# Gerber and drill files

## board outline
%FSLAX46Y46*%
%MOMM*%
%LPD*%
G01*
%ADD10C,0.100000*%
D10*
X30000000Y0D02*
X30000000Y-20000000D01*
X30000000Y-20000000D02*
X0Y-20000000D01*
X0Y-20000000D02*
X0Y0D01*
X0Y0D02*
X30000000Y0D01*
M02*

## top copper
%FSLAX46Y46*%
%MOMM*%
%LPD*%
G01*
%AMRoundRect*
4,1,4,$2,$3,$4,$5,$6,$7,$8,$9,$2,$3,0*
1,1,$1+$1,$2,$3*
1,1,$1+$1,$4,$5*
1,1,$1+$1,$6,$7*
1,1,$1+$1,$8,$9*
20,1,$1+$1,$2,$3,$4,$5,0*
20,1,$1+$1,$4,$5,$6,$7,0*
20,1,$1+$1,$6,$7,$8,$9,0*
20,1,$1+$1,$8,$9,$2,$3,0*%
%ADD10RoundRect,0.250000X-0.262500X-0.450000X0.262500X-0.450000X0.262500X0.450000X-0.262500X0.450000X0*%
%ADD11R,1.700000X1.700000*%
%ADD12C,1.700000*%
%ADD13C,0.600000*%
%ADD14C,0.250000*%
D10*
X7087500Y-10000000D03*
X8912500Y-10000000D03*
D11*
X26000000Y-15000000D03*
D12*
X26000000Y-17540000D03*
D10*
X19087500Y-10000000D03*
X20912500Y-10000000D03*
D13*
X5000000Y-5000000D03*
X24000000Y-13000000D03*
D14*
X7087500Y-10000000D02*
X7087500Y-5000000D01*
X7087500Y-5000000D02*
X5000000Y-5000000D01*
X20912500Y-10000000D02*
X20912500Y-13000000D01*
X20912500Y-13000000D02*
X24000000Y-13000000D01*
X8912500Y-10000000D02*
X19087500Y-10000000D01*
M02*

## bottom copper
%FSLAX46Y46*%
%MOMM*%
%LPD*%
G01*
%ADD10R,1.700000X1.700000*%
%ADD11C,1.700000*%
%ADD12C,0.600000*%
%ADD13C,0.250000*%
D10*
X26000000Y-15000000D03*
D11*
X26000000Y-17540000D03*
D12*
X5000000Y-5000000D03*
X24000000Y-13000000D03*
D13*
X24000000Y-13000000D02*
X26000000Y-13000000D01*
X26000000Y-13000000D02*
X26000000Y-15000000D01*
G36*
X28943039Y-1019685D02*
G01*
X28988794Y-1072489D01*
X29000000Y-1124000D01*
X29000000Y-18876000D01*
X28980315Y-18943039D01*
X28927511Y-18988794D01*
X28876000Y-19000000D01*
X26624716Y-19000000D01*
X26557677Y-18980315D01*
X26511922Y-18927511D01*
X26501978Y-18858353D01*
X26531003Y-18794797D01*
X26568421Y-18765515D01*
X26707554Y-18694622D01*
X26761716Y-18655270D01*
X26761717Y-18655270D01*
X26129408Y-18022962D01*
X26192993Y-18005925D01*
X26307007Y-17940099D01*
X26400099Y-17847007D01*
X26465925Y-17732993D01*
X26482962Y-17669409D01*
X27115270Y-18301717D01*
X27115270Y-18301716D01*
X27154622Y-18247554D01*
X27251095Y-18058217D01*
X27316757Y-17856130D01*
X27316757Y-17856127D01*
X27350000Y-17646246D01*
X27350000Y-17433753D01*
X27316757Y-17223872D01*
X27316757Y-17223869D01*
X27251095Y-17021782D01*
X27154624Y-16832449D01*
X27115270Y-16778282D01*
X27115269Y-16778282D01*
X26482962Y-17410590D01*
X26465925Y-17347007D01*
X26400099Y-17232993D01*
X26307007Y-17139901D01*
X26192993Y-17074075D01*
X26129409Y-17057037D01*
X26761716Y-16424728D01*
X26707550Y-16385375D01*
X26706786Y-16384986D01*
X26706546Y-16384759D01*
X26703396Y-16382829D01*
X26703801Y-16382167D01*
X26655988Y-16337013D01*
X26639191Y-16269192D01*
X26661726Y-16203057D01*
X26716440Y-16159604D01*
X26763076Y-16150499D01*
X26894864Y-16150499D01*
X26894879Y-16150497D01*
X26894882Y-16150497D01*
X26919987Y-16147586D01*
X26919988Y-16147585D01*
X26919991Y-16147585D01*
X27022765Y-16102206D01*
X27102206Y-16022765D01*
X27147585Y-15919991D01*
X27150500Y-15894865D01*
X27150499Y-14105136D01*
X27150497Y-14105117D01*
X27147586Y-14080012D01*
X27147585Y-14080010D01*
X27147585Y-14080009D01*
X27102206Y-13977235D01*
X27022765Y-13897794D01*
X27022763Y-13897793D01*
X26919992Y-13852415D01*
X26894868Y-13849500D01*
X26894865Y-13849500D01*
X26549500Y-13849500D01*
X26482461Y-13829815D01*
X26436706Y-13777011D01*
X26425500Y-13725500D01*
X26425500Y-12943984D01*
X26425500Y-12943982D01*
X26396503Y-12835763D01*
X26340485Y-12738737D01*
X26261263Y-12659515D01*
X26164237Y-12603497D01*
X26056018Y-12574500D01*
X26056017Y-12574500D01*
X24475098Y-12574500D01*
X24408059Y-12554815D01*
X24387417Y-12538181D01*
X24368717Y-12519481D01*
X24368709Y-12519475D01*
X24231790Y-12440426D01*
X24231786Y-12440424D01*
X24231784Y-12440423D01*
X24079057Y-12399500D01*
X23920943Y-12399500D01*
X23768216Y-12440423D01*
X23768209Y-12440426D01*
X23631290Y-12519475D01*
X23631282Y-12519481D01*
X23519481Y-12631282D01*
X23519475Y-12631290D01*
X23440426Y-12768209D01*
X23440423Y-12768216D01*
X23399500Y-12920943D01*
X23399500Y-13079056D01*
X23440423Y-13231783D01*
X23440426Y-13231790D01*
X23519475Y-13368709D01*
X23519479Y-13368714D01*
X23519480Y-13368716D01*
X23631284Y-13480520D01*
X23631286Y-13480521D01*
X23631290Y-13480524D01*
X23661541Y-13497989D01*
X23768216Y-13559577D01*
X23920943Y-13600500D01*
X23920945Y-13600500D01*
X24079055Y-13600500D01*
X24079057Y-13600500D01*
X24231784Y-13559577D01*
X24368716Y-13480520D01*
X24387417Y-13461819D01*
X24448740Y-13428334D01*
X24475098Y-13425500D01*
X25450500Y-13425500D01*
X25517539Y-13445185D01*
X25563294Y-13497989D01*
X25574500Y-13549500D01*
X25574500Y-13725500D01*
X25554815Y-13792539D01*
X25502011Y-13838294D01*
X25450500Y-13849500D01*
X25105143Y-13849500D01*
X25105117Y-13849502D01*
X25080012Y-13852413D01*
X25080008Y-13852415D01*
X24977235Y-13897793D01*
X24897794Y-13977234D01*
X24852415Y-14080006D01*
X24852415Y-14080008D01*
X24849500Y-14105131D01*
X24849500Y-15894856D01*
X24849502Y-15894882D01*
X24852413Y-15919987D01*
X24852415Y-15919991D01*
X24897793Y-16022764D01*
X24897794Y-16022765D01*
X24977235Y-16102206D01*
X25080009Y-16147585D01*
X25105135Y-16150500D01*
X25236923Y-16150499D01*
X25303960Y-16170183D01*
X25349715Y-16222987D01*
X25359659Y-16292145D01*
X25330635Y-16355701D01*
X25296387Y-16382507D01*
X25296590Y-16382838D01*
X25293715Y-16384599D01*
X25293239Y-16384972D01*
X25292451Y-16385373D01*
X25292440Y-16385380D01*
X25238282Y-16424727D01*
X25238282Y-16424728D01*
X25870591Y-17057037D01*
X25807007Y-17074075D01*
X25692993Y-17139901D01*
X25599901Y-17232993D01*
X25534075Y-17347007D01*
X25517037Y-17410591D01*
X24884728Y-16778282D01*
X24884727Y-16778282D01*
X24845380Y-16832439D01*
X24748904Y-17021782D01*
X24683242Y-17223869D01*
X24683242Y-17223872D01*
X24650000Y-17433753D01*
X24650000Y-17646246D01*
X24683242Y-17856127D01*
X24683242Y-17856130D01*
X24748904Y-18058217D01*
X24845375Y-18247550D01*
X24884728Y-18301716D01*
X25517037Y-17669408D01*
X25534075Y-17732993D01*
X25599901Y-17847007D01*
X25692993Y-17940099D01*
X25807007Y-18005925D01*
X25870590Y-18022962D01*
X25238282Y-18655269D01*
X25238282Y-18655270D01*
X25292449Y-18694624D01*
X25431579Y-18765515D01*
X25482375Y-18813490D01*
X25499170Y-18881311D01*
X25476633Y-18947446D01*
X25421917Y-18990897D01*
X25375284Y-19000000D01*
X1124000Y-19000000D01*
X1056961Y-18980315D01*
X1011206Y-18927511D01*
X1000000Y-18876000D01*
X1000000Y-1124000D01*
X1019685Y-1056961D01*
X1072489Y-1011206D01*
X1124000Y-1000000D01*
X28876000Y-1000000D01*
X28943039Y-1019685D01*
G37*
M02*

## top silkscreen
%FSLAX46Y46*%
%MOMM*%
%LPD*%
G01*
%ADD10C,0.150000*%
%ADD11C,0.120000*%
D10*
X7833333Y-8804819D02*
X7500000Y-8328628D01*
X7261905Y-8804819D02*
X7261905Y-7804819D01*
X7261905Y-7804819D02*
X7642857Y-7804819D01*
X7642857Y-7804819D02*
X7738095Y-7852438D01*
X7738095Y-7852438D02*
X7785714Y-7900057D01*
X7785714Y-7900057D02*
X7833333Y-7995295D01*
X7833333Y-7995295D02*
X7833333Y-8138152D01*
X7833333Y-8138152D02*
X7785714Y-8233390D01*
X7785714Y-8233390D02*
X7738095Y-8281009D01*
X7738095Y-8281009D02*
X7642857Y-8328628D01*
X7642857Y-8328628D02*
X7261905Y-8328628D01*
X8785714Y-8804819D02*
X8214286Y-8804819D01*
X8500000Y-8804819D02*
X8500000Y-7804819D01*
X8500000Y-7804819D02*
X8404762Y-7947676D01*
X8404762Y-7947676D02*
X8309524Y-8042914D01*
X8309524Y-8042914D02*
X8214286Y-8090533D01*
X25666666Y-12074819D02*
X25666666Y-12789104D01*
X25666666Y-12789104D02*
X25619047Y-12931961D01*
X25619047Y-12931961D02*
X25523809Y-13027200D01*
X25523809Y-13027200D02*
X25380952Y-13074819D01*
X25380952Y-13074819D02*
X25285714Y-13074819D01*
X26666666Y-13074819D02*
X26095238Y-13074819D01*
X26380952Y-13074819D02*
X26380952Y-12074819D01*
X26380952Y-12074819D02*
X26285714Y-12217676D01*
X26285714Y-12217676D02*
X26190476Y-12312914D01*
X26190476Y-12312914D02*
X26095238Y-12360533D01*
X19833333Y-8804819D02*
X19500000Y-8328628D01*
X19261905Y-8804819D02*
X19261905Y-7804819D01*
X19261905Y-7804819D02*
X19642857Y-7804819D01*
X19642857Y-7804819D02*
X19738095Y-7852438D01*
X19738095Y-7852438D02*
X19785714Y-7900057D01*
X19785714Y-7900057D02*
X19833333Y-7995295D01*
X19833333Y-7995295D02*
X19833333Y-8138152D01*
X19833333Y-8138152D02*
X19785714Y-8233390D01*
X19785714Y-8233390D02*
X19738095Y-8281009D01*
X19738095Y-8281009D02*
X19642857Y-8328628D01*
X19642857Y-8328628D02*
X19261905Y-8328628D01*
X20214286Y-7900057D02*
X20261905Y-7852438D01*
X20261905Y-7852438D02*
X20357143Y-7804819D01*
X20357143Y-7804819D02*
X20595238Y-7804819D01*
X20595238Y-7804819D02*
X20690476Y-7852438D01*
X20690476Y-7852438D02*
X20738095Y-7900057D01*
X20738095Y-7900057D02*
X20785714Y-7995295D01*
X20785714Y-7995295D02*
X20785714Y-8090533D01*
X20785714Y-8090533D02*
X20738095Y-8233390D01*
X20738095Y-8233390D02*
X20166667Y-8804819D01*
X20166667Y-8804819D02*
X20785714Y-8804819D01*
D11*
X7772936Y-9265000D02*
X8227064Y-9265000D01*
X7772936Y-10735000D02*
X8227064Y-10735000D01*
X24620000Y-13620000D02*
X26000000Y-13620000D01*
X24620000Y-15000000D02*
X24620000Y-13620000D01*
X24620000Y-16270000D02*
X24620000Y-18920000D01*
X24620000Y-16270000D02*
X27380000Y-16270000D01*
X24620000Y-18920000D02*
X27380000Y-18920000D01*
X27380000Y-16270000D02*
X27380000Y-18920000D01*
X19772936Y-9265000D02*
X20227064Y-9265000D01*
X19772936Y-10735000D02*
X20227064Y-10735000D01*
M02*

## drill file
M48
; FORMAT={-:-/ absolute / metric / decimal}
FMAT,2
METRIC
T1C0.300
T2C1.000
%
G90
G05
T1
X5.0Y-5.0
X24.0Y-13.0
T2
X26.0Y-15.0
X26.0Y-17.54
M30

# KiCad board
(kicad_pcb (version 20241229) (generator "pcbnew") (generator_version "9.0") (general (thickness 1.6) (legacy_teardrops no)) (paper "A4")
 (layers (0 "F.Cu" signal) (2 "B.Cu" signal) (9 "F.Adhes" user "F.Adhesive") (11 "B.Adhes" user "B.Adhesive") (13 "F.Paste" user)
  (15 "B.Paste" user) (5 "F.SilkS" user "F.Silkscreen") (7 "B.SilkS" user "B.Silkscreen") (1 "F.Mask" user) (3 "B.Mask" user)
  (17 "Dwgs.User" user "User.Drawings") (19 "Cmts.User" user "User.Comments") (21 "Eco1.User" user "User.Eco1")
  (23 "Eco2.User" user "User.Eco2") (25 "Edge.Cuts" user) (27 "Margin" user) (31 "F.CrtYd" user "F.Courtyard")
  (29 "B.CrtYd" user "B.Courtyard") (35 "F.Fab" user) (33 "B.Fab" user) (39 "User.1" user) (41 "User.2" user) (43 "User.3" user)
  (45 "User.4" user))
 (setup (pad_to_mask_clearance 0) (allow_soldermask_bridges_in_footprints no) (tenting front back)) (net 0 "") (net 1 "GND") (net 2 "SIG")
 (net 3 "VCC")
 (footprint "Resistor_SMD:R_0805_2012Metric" (layer "F.Cu") (at 8 10)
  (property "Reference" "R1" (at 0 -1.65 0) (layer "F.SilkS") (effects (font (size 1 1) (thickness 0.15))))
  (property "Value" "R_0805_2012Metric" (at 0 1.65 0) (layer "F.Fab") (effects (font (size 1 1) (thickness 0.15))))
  (fp_line (start -0.227064 -0.735) (end 0.227064 -0.735) (stroke (width 0.12) (type solid)) (layer "F.SilkS"))
  (fp_line (start -0.227064 0.735) (end 0.227064 0.735) (stroke (width 0.12) (type solid)) (layer "F.SilkS"))
  (pad "1" smd roundrect (at -0.9125 0) (size 1.025 1.4) (layers "F.Cu" "F.Mask" "F.Paste") (roundrect_rratio 0.243902) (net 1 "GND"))
  (pad "2" smd roundrect (at 0.9125 0) (size 1.025 1.4) (layers "F.Cu" "F.Mask" "F.Paste") (roundrect_rratio 0.243902) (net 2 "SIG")))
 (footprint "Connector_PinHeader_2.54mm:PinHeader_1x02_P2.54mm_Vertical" (layer "F.Cu") (at 26 15)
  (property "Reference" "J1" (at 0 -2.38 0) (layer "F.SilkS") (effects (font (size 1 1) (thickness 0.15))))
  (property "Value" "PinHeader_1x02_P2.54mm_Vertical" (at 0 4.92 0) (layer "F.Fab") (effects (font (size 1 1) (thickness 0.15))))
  (fp_line (start -1.38 -1.38) (end 0 -1.38) (stroke (width 0.12) (type solid)) (layer "F.SilkS"))
  (fp_line (start -1.38 0) (end -1.38 -1.38) (stroke (width 0.12) (type solid)) (layer "F.SilkS"))
  (fp_line (start -1.38 1.27) (end -1.38 3.92) (stroke (width 0.12) (type solid)) (layer "F.SilkS"))
  (fp_line (start -1.38 1.27) (end 1.38 1.27) (stroke (width 0.12) (type solid)) (layer "F.SilkS"))
  (fp_line (start -1.38 3.92) (end 1.38 3.92) (stroke (width 0.12) (type solid)) (layer "F.SilkS"))
  (fp_line (start 1.38 1.27) (end 1.38 3.92) (stroke (width 0.12) (type solid)) (layer "F.SilkS"))
  (pad "1" thru_hole rect (at 0 0) (size 1.7 1.7) (drill 1) (layers "*.Cu" "*.Mask") (remove_unused_layers no) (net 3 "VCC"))
  (pad "2" thru_hole circle (at 0 2.54) (size 1.7 1.7) (drill 1) (layers "*.Cu" "*.Mask") (remove_unused_layers no) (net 1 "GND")))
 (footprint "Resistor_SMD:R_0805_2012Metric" (layer "F.Cu") (at 20 10)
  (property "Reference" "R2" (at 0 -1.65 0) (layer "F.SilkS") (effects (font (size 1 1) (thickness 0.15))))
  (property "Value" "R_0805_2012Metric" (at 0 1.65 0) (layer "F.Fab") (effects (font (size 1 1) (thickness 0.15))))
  (fp_line (start -0.227064 -0.735) (end 0.227064 -0.735) (stroke (width 0.12) (type solid)) (layer "F.SilkS"))
  (fp_line (start -0.227064 0.735) (end 0.227064 0.735) (stroke (width 0.12) (type solid)) (layer "F.SilkS"))
  (pad "1" smd roundrect (at -0.9125 0) (size 1.025 1.4) (layers "F.Cu" "F.Mask" "F.Paste") (roundrect_rratio 0.243902) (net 2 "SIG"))
  (pad "2" smd roundrect (at 0.9125 0) (size 1.025 1.4) (layers "F.Cu" "F.Mask" "F.Paste") (roundrect_rratio 0.243902) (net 3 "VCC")))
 (gr_line (start 30 0) (end 30 20) (stroke (width 0.1) (type default)) (layer "Edge.Cuts"))
 (gr_line (start 30 20) (end 0 20) (stroke (width 0.1) (type default)) (layer "Edge.Cuts"))
 (gr_line (start 0 20) (end 0 0) (stroke (width 0.1) (type default)) (layer "Edge.Cuts"))
 (gr_line (start 0 0) (end 30 0) (stroke (width 0.1) (type default)) (layer "Edge.Cuts"))
 (segment (start 7.0875 10) (end 7.0875 5) (width 0.25) (layer "F.Cu") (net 1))
 (segment (start 7.0875 5) (end 5 5) (width 0.25) (layer "F.Cu") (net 1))
 (via (at 5 5) (size 0.6) (drill 0.3) (layers "F.Cu" "B.Cu") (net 1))
 (segment (start 20.9125 10) (end 20.9125 13) (width 0.25) (layer "F.Cu") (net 3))
 (segment (start 20.9125 13) (end 24 13) (width 0.25) (layer "F.Cu") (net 3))
 (via (at 24 13) (size 0.6) (drill 0.3) (layers "F.Cu" "B.Cu") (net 3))
 (segment (start 24 13) (end 26 13) (width 0.25) (layer "B.Cu") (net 3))
 (segment (start 26 13) (end 26 15) (width 0.25) (layer "B.Cu") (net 3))
 (segment (start 8.9125 10) (end 19.0875 10) (width 0.25) (layer "F.Cu") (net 2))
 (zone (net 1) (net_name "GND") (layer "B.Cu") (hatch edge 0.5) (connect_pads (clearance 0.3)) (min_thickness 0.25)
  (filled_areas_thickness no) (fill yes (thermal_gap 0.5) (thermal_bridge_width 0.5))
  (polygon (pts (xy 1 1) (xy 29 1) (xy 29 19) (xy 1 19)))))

